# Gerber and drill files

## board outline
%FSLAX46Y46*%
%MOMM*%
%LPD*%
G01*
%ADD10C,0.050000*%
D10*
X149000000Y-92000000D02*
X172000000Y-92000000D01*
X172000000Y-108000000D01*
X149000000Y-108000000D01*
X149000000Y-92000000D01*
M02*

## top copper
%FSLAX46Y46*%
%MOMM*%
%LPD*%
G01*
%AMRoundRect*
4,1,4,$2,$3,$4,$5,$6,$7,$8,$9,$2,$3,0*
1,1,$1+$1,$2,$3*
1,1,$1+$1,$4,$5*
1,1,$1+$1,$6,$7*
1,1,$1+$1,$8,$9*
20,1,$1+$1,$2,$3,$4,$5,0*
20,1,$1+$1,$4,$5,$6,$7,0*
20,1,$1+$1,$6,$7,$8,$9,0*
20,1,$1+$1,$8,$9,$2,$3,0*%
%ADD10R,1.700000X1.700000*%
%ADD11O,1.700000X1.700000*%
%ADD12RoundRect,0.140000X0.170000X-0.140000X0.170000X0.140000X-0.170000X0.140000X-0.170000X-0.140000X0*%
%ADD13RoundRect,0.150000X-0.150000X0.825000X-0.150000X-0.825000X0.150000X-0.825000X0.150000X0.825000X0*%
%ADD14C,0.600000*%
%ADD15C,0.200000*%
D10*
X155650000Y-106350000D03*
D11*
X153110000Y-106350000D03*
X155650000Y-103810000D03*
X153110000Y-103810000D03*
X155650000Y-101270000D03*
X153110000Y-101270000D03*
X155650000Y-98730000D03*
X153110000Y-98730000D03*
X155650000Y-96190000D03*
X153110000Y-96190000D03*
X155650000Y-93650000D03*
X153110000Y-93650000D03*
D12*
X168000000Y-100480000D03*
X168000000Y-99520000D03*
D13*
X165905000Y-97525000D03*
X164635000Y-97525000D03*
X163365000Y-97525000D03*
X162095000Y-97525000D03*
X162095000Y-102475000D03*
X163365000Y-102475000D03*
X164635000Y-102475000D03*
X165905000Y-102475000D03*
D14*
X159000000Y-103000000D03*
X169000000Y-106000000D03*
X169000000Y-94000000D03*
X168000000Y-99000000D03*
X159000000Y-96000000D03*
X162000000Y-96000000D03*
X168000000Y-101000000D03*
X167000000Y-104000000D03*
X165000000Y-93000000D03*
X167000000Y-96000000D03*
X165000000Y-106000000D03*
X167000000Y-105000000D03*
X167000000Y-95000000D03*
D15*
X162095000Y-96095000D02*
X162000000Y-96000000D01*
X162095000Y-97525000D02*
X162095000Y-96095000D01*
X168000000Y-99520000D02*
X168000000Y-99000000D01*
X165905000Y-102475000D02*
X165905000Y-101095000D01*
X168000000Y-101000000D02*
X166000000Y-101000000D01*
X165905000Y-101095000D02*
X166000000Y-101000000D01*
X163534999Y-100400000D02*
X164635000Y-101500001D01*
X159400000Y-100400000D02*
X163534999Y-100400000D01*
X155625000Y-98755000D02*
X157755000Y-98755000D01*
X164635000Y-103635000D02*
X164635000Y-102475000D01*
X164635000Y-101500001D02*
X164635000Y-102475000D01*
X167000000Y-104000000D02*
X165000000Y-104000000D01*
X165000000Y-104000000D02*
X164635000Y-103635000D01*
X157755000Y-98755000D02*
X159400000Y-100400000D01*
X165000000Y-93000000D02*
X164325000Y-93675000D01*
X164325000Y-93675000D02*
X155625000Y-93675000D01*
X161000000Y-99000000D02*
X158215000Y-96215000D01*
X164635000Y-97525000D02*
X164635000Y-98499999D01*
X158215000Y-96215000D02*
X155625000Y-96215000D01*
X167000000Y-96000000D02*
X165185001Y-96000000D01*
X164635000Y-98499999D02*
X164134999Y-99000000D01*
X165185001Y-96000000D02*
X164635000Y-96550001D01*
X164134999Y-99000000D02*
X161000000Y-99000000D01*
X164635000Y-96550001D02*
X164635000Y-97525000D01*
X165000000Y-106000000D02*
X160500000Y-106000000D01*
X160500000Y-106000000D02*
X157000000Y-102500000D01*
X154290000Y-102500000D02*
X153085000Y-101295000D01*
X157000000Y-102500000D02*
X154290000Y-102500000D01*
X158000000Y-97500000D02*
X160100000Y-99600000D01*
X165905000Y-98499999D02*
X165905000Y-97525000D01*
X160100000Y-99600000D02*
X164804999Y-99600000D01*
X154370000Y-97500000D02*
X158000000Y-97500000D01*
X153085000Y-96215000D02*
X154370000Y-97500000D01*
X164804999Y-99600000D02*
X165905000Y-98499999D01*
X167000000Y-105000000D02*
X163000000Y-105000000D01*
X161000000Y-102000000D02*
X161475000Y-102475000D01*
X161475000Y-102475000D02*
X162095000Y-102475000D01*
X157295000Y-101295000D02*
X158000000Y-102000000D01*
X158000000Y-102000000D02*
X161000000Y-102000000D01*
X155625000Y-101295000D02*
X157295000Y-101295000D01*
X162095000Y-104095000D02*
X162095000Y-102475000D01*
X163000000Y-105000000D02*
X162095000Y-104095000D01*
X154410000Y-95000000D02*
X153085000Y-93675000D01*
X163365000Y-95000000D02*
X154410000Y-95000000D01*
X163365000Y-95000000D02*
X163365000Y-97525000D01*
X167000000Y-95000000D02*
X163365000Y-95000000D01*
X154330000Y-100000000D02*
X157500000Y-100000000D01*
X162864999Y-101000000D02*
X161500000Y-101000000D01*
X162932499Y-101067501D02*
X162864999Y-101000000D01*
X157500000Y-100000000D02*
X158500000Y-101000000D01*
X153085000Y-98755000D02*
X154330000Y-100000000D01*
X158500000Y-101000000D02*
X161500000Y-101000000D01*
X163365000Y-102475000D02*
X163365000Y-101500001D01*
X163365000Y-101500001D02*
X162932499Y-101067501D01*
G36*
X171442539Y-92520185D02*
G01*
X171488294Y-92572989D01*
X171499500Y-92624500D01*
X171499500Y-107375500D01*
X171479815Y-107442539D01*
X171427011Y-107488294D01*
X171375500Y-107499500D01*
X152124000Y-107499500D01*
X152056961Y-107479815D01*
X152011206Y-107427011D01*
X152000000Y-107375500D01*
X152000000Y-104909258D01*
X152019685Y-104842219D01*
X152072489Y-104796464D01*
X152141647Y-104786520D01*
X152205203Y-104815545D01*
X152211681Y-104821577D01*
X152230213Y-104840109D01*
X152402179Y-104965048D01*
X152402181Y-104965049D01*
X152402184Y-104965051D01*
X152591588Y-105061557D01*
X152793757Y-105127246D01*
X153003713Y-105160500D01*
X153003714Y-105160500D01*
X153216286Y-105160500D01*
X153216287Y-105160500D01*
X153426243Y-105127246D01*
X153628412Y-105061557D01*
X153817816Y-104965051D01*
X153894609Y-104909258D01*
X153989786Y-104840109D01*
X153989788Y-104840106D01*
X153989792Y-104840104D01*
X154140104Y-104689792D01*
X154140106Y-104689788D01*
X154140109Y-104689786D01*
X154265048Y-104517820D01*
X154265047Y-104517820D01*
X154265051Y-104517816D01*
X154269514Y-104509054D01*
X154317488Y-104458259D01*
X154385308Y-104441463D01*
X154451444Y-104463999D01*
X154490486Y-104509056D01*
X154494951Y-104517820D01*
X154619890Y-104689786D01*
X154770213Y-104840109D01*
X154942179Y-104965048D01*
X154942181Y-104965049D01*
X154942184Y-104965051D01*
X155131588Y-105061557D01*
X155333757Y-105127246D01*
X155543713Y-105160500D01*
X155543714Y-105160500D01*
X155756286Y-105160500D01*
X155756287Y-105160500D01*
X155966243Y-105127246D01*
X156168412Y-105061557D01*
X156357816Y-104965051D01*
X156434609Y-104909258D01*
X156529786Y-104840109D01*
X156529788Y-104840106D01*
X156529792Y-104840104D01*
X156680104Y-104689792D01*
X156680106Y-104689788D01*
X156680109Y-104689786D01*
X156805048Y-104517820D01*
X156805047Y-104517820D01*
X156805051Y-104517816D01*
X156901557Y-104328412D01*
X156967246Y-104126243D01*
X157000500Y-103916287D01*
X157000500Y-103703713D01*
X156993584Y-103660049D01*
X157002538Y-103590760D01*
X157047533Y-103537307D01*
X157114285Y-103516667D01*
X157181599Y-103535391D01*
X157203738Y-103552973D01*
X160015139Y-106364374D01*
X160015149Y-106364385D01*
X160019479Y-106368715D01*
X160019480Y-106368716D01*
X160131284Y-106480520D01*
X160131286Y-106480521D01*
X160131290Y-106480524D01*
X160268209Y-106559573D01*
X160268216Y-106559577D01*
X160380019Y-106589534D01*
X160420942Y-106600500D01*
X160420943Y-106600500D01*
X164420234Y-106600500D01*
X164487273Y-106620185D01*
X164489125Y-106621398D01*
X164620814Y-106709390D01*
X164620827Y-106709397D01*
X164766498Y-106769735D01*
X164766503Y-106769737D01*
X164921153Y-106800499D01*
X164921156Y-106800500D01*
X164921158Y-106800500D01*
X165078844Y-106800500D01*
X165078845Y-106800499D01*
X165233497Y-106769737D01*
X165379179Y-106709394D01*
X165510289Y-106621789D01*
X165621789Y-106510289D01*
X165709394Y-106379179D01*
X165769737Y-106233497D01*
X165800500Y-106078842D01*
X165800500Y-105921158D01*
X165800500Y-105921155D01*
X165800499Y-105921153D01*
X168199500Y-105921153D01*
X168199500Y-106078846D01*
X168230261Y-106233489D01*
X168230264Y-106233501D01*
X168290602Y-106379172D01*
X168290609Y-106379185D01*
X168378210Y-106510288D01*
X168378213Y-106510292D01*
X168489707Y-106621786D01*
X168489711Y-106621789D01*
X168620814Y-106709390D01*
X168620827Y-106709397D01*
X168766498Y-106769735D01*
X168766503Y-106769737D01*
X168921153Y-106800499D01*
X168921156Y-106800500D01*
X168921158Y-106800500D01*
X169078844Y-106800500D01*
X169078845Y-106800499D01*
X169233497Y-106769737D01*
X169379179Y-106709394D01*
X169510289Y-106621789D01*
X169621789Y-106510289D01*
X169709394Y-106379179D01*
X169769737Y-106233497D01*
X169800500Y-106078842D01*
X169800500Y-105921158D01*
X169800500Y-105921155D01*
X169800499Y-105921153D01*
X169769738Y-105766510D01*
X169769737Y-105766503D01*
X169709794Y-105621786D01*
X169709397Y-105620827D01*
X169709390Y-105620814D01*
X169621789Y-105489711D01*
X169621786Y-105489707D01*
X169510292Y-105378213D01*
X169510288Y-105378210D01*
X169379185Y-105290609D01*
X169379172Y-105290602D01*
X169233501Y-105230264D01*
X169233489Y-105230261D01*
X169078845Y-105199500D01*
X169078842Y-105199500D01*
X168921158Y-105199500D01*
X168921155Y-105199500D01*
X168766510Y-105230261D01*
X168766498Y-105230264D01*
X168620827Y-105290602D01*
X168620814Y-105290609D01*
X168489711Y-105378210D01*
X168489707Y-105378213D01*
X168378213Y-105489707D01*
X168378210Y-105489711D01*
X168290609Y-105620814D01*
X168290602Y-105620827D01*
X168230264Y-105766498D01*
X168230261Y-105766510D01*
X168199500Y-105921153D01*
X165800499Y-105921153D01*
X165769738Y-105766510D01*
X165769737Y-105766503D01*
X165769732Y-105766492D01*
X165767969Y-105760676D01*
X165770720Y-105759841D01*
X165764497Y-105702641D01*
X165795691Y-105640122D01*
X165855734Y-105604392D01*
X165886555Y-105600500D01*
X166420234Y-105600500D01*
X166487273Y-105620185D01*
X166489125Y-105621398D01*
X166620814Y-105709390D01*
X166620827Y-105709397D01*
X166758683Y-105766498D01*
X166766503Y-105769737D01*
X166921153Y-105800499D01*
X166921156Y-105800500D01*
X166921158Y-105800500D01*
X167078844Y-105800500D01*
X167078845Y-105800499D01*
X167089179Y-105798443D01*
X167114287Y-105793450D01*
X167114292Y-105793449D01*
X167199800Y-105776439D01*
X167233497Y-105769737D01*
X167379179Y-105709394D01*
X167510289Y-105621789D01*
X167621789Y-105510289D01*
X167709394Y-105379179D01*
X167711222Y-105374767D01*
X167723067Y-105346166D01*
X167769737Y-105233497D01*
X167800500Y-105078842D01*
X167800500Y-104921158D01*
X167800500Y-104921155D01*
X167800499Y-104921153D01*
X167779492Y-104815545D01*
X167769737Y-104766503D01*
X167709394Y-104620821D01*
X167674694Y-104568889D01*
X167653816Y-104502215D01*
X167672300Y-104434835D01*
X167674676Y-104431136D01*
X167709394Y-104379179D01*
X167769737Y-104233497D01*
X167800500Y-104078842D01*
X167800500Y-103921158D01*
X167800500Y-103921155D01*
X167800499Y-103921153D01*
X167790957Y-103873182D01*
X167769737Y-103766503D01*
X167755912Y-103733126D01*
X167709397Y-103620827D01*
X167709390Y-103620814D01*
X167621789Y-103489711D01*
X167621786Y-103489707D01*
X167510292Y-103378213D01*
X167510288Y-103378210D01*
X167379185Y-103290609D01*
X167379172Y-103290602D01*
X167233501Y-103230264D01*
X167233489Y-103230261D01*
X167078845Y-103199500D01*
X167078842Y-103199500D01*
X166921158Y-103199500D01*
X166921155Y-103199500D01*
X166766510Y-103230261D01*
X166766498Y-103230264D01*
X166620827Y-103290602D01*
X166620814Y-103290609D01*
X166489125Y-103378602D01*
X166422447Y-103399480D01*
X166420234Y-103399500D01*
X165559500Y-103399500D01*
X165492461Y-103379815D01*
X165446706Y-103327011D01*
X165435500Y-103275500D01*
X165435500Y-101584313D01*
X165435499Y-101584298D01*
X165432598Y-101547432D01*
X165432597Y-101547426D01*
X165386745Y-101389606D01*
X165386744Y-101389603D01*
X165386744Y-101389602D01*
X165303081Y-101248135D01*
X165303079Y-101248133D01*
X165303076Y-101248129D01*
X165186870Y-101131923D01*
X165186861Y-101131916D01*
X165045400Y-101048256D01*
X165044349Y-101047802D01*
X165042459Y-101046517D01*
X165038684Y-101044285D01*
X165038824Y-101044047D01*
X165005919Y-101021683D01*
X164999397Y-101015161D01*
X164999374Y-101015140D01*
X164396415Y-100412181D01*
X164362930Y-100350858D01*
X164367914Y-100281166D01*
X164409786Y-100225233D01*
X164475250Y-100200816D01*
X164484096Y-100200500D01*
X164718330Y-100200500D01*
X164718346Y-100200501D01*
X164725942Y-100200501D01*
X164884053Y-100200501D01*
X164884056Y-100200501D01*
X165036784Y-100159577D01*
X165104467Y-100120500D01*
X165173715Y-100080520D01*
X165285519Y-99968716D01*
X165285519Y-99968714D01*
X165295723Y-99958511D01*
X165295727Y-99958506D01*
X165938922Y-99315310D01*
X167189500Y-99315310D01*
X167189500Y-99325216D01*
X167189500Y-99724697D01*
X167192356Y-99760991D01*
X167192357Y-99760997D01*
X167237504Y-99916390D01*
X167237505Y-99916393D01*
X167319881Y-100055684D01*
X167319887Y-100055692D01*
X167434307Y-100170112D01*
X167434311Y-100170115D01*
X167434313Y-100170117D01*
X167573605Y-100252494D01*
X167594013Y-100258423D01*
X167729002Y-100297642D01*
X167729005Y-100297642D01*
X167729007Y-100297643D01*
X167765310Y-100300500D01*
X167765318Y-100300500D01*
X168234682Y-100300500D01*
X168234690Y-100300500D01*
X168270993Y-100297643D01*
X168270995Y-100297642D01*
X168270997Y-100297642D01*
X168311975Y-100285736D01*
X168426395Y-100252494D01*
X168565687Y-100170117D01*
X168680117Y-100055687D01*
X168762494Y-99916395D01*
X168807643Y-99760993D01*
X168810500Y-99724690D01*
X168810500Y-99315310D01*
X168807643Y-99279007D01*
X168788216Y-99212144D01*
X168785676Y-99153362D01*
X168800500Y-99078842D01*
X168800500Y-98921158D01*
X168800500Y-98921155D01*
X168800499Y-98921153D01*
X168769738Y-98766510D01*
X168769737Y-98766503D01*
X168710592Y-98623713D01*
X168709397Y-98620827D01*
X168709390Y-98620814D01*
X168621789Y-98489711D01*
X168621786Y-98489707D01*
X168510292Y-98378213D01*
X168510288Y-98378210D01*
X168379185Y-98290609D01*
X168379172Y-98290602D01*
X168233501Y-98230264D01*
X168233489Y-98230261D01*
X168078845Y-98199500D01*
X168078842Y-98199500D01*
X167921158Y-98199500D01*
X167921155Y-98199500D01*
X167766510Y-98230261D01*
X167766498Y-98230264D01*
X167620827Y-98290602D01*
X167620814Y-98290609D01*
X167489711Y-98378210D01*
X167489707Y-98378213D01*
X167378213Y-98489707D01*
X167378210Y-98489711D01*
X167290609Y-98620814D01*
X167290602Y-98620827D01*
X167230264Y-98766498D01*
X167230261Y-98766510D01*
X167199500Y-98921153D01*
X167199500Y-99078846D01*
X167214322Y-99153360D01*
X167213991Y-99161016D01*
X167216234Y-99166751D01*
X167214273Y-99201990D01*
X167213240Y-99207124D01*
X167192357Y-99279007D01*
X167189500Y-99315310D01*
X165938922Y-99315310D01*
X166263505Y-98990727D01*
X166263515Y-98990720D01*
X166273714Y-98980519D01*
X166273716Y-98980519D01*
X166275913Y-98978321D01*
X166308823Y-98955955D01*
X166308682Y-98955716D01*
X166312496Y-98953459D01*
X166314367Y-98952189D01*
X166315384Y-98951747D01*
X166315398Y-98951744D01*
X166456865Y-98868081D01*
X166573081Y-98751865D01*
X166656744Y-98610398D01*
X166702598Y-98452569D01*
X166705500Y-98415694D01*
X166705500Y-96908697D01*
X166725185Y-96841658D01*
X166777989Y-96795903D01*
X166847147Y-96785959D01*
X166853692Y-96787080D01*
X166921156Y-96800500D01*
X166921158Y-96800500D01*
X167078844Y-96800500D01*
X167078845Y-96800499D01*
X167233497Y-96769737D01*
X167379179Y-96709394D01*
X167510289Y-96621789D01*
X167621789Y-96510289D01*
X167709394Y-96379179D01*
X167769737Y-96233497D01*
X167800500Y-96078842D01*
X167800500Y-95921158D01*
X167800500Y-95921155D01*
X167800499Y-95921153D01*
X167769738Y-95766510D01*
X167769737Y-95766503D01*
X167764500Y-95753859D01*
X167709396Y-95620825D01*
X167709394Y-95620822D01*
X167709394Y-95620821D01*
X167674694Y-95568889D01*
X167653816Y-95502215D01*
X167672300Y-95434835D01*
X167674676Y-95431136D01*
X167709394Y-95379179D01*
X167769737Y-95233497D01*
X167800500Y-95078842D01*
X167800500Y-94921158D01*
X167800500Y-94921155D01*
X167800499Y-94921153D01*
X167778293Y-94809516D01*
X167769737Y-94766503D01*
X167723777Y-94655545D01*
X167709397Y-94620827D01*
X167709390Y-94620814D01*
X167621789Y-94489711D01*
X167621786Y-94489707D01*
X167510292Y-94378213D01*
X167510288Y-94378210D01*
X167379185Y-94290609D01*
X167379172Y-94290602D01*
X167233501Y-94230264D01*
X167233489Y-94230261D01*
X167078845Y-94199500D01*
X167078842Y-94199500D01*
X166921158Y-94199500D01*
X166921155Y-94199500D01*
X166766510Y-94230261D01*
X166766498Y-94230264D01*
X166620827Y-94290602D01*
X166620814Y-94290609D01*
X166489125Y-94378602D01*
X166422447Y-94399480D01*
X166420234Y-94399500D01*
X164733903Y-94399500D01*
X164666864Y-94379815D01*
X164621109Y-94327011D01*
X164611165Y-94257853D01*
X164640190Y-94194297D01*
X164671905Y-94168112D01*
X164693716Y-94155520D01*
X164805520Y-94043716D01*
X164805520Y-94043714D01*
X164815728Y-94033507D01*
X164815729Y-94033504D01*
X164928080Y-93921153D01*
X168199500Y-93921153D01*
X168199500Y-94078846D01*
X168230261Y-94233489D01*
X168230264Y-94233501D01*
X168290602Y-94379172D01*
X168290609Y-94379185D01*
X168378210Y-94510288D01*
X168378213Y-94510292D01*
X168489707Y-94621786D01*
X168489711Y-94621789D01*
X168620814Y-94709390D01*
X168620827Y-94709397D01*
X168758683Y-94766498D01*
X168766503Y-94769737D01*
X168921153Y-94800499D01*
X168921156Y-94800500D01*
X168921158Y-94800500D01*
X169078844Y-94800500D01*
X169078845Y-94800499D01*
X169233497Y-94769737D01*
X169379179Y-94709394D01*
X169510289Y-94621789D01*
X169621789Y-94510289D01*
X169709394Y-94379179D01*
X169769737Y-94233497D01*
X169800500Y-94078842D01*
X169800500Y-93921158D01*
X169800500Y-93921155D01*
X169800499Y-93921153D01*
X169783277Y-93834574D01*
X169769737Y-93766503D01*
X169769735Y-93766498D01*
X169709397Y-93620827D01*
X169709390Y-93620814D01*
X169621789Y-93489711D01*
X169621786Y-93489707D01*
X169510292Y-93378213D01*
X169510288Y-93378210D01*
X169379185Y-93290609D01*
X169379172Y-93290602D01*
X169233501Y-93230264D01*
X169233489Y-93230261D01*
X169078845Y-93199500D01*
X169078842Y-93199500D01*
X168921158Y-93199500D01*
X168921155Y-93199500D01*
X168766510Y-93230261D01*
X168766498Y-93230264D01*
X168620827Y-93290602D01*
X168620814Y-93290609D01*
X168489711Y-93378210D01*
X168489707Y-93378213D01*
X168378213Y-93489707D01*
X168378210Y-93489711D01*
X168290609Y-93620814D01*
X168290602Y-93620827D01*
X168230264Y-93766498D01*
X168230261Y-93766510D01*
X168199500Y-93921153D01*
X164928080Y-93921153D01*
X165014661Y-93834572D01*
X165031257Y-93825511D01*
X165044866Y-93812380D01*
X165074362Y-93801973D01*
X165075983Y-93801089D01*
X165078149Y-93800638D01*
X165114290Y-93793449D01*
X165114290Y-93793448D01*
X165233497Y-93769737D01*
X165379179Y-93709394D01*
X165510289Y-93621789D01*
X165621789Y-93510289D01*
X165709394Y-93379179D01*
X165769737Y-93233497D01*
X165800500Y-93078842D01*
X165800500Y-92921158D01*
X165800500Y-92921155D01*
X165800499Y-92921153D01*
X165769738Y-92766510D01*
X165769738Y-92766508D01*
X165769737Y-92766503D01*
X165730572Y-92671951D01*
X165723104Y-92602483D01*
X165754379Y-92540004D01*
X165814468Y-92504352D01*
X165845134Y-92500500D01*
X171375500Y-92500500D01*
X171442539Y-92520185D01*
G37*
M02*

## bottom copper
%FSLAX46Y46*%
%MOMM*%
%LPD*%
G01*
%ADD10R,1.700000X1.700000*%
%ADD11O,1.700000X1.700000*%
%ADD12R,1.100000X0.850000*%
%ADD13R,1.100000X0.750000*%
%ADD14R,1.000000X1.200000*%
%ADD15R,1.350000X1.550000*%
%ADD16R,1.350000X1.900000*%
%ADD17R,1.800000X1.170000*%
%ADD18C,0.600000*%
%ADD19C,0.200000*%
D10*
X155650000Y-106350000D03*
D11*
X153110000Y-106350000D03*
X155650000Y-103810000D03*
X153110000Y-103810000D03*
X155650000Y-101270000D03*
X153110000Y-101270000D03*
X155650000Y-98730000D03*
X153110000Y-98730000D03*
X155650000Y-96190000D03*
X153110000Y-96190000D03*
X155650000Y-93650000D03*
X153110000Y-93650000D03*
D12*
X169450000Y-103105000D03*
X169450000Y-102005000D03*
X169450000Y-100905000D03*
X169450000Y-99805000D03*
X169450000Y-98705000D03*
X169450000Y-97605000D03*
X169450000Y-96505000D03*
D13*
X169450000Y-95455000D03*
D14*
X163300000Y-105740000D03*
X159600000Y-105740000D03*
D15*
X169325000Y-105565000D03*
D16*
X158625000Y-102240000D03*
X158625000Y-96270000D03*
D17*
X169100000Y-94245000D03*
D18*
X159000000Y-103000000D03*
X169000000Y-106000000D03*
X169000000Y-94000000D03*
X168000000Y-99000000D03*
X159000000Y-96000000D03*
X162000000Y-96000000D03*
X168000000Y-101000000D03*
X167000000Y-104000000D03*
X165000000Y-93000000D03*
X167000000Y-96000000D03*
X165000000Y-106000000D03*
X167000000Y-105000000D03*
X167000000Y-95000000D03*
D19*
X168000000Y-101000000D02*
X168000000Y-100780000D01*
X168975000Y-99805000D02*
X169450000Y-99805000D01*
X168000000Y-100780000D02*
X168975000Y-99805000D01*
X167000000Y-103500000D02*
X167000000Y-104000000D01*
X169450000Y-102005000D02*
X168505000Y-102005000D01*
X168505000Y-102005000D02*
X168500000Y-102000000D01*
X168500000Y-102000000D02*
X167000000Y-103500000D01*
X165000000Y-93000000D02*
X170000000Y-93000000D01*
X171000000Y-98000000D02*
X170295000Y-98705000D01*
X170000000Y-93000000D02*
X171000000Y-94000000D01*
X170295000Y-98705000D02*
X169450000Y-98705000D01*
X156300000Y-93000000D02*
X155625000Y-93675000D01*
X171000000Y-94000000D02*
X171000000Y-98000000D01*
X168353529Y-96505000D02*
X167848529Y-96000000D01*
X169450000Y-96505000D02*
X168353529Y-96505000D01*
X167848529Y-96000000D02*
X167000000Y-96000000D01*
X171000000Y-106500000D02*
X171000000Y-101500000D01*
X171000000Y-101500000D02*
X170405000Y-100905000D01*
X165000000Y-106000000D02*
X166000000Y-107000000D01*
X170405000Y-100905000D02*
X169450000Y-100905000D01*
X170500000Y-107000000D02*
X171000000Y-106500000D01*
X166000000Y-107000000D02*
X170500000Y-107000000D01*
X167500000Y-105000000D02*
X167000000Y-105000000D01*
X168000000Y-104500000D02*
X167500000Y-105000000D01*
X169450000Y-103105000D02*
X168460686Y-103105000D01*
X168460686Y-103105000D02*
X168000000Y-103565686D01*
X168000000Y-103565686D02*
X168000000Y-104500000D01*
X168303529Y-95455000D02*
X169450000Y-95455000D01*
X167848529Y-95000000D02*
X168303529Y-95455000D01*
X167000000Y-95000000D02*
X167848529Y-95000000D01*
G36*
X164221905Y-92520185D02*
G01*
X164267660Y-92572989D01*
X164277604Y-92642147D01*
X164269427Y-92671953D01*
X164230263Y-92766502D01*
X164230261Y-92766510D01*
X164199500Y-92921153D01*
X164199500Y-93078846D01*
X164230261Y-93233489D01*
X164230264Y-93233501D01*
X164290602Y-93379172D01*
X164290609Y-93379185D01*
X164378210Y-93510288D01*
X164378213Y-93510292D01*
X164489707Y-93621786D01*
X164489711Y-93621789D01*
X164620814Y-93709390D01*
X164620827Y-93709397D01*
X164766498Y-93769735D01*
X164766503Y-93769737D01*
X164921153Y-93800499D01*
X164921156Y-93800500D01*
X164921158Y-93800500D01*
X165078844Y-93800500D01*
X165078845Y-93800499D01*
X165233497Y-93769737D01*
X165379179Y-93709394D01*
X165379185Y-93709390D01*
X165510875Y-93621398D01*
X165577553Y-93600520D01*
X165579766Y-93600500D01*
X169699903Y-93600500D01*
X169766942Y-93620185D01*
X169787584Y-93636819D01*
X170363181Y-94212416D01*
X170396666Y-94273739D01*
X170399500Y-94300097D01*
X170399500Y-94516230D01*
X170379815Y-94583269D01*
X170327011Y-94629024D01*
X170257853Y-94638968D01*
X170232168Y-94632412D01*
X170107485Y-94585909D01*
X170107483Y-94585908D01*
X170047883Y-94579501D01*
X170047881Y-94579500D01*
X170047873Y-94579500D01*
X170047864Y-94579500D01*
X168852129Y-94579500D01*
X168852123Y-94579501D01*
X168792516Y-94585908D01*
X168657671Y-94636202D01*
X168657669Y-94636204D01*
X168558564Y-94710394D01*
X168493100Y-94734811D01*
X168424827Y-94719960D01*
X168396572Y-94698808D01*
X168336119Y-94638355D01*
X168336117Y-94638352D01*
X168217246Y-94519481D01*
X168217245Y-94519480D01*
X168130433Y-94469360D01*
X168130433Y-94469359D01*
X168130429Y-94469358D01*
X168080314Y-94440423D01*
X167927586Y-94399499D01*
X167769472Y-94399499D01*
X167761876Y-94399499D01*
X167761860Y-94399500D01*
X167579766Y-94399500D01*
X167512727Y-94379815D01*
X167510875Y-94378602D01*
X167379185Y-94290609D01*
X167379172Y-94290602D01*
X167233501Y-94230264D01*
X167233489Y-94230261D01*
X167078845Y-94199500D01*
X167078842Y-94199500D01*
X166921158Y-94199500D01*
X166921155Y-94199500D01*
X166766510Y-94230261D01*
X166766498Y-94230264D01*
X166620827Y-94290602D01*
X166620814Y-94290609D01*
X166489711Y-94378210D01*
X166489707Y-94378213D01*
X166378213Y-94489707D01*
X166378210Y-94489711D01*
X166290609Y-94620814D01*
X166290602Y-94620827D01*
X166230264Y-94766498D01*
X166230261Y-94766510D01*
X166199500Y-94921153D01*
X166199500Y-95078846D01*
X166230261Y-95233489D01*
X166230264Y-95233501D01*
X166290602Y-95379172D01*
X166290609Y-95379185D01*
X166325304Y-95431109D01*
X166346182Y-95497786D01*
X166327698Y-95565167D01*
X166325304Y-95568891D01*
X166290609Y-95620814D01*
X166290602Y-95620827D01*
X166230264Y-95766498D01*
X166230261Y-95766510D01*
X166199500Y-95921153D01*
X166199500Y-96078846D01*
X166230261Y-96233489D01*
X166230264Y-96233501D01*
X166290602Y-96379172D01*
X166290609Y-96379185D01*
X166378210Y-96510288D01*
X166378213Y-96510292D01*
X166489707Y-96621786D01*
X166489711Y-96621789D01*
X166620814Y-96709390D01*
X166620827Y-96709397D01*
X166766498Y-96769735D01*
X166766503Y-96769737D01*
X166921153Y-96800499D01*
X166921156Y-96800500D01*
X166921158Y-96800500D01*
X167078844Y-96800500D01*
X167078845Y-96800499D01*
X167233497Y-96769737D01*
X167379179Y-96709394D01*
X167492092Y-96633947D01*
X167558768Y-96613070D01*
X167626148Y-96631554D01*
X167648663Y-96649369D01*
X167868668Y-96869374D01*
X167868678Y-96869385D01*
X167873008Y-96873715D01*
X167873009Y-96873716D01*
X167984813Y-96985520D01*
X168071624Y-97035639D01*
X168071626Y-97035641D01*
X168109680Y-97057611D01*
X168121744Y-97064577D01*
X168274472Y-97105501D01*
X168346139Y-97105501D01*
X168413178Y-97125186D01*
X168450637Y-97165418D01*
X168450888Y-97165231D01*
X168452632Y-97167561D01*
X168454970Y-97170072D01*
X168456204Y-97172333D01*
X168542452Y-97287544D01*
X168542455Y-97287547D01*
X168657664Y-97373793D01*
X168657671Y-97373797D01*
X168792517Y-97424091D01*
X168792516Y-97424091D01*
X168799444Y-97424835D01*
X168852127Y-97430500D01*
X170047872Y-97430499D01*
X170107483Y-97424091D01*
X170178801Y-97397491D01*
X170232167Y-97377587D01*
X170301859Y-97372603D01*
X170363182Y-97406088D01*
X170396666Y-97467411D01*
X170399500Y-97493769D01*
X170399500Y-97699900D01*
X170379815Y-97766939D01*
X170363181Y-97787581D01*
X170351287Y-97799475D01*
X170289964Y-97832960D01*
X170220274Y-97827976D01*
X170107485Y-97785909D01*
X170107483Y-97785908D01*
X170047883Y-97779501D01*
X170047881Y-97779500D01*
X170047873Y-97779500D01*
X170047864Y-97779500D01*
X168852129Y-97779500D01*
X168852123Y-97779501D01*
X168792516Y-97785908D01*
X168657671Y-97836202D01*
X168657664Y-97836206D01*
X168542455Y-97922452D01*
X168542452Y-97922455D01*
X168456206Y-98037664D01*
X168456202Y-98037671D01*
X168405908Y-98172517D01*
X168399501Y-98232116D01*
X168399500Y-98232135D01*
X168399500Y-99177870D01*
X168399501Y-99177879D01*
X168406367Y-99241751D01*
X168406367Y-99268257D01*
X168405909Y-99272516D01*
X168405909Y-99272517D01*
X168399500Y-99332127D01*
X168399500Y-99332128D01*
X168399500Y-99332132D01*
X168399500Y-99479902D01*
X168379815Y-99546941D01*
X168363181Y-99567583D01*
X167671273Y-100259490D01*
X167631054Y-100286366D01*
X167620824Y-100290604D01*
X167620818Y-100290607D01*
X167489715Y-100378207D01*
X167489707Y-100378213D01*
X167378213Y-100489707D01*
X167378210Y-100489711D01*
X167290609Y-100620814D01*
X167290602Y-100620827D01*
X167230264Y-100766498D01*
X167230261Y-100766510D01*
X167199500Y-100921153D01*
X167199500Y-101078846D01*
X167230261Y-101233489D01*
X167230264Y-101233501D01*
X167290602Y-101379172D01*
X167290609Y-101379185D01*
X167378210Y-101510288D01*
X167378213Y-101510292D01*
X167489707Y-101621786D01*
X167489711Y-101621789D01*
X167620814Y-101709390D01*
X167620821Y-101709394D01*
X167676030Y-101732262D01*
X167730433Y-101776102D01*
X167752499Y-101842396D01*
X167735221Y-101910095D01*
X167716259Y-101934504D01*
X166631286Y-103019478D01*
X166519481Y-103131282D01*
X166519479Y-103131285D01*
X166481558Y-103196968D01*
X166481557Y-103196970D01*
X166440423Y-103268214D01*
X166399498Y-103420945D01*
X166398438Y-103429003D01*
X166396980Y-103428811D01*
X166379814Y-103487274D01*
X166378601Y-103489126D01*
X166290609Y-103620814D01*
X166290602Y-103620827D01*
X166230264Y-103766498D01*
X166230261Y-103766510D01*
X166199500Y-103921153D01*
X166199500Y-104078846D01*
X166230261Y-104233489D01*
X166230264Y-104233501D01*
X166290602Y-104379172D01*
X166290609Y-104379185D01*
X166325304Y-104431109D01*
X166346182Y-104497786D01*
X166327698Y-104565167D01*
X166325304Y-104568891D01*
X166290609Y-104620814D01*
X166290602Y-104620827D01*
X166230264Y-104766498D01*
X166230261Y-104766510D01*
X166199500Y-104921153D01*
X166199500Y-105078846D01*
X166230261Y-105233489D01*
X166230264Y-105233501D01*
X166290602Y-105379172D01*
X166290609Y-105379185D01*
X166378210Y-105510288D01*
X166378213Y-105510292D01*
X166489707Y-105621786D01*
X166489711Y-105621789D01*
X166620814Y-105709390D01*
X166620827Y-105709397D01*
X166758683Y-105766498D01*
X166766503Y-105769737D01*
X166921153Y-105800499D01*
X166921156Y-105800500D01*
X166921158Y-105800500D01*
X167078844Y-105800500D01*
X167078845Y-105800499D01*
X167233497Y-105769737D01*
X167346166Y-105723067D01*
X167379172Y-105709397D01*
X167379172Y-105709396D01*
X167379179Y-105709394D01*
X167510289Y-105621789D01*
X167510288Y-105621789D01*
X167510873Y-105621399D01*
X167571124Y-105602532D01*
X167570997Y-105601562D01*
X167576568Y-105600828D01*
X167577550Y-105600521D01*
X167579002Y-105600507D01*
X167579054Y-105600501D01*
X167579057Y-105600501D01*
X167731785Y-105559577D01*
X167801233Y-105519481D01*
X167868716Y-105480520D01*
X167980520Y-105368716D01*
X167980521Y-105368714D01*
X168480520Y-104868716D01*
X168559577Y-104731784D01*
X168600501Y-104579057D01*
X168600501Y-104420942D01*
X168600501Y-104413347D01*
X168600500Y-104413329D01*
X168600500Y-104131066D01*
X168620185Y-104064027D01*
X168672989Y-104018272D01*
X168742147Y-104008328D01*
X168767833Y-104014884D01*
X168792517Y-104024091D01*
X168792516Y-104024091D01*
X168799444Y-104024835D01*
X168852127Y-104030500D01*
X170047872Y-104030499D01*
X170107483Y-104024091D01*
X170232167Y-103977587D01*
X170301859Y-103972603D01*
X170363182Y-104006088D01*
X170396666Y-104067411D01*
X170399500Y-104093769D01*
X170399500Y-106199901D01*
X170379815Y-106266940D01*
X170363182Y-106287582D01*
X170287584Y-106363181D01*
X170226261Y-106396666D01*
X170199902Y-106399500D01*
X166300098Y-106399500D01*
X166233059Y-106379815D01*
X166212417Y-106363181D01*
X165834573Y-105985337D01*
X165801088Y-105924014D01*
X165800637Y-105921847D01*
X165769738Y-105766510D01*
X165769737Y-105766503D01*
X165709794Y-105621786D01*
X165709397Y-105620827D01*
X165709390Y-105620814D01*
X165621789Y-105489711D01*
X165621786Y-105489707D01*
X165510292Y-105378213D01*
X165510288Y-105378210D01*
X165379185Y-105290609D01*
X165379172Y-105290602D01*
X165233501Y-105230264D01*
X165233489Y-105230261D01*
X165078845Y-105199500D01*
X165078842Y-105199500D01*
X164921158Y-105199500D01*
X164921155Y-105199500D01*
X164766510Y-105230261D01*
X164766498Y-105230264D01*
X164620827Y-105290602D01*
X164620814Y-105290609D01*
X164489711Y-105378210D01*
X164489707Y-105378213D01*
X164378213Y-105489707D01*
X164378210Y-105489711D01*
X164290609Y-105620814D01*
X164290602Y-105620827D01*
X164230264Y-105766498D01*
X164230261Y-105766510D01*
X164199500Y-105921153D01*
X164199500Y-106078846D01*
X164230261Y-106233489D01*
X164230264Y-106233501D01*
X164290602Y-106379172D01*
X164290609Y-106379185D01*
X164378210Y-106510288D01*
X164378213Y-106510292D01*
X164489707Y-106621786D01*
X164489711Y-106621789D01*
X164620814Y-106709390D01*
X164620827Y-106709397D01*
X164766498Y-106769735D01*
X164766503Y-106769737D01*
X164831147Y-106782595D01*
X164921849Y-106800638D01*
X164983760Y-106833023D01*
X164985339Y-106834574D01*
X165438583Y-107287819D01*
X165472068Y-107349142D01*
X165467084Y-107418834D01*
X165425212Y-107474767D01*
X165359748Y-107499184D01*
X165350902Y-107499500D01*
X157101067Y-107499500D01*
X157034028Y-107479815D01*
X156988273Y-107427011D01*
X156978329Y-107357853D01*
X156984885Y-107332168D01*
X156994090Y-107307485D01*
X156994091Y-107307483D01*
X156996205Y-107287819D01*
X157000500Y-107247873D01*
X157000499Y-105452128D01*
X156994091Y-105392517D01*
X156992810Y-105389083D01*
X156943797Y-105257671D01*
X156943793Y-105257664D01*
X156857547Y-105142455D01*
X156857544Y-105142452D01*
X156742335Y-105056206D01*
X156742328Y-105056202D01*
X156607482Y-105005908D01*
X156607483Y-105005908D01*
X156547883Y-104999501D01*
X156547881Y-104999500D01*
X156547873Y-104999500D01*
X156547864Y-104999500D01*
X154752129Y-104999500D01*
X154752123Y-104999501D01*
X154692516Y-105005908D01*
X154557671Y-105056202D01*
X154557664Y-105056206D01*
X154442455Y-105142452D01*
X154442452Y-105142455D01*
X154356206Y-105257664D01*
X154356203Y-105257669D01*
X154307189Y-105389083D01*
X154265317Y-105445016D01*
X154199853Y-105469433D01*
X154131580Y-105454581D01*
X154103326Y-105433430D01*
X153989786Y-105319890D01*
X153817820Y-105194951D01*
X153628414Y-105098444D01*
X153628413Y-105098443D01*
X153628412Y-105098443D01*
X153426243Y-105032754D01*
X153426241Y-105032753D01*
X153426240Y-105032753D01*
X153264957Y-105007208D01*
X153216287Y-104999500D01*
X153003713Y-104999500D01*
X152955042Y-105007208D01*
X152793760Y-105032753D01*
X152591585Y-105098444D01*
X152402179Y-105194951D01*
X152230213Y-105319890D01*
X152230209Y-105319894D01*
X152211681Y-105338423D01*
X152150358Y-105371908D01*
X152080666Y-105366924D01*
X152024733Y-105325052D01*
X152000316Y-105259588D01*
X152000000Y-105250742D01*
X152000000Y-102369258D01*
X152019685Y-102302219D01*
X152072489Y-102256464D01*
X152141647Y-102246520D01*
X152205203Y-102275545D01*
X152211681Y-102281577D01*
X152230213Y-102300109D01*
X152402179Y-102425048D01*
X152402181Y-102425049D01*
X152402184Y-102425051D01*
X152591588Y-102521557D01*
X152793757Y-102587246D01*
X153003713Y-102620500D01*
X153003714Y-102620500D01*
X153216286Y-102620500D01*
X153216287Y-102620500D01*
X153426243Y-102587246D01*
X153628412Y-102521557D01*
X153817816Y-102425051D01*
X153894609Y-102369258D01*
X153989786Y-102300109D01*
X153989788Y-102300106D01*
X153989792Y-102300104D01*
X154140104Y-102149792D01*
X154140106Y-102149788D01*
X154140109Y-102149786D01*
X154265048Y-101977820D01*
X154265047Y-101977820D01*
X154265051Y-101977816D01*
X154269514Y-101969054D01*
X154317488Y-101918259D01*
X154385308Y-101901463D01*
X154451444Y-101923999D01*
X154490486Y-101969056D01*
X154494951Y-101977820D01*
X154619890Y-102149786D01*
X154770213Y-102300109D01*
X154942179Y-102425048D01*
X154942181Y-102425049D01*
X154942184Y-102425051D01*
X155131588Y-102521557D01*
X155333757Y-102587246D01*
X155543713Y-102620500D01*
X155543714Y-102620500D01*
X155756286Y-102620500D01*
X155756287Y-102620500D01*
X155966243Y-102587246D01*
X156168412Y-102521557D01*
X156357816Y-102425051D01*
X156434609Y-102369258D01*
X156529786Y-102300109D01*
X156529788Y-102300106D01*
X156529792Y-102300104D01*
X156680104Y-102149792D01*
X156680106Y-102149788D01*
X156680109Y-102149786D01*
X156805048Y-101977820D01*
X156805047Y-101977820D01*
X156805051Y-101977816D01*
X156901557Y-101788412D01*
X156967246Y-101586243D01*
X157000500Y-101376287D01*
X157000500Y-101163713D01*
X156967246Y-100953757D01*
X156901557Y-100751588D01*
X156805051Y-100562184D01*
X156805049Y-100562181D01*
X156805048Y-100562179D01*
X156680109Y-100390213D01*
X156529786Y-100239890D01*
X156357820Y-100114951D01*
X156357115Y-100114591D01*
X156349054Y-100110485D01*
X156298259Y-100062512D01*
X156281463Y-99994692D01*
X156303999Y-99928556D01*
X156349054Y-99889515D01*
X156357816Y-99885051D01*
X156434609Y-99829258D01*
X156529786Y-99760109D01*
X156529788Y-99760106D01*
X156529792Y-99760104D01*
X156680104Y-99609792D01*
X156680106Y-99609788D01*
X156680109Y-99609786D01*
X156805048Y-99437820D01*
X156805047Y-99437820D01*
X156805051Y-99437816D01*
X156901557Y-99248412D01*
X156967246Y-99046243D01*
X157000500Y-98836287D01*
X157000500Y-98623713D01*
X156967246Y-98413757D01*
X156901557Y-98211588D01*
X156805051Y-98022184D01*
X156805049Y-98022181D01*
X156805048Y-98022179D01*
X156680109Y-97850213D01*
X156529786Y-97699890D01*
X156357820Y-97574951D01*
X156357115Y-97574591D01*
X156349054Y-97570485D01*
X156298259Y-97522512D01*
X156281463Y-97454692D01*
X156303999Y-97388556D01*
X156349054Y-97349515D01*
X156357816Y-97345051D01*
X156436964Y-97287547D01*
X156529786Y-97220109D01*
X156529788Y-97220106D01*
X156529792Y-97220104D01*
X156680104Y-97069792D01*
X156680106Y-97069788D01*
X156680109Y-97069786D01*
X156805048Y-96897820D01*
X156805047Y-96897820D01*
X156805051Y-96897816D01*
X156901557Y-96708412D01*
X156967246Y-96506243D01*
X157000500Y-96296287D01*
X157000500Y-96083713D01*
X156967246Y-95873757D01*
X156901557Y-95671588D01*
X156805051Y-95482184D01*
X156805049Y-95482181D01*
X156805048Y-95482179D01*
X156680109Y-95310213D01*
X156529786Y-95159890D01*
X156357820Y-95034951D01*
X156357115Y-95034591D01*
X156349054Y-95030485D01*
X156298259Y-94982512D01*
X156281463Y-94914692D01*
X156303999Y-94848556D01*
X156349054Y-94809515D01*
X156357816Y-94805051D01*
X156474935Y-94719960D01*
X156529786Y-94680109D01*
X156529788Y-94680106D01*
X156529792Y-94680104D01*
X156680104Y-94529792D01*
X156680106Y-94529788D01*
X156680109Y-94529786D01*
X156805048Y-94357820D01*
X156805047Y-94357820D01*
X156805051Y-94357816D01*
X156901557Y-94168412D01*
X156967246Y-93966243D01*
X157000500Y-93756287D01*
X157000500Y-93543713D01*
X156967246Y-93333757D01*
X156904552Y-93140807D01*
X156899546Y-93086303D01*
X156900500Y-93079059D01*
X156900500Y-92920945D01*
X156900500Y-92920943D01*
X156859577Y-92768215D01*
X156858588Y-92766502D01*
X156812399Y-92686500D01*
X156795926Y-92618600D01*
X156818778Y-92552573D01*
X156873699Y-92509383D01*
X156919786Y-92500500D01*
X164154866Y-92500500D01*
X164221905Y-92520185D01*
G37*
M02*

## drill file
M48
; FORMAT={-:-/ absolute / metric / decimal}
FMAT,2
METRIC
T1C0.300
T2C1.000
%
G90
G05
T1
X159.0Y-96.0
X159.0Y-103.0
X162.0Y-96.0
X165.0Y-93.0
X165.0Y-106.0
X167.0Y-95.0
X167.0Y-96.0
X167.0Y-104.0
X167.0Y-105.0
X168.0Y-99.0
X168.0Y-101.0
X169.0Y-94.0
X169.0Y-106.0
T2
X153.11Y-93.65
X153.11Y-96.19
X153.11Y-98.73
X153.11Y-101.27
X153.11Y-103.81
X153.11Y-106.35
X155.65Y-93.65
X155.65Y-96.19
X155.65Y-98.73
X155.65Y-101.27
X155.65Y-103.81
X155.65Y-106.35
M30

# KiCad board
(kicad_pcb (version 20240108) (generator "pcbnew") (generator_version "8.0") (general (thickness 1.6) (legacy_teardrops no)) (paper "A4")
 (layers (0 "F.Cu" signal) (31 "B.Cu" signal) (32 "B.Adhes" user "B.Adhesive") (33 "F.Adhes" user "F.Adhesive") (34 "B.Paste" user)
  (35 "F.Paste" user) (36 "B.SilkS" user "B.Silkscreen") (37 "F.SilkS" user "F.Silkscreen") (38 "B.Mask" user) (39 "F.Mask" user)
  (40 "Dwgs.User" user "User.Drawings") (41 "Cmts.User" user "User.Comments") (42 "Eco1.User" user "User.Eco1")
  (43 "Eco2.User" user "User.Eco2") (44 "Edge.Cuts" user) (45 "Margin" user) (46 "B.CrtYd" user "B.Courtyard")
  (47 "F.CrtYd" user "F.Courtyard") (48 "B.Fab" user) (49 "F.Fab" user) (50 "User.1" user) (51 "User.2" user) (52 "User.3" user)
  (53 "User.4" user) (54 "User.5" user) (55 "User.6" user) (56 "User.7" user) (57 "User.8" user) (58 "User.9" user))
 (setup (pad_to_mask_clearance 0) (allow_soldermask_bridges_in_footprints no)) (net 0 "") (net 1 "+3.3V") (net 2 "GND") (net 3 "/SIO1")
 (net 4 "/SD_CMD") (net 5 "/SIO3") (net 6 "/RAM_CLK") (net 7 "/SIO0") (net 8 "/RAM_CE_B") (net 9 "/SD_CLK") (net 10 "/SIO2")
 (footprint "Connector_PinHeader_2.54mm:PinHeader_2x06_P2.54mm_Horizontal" (layer "F.Cu") (at 155.65 106.35 180)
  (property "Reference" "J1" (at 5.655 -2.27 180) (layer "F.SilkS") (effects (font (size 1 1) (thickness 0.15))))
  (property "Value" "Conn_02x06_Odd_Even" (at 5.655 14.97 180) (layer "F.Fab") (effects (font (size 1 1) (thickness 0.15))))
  (pad "1" thru_hole rect (at 0 0 180) (size 1.7 1.7) (drill 1) (layers "*.Cu" "*.Mask") (remove_unused_layers no) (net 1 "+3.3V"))
  (pad "2" thru_hole oval (at 2.54 0 180) (size 1.7 1.7) (drill 1) (layers "*.Cu" "*.Mask") (remove_unused_layers no) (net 1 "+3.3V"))
  (pad "3" thru_hole oval (at 0 2.54 180) (size 1.7 1.7) (drill 1) (layers "*.Cu" "*.Mask") (remove_unused_layers no) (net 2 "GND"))
  (pad "4" thru_hole oval (at 2.54 2.54 180) (size 1.7 1.7) (drill 1) (layers "*.Cu" "*.Mask") (remove_unused_layers no) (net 2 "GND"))
  (pad "5" thru_hole oval (at 0 5.08 180) (size 1.7 1.7) (drill 1) (layers "*.Cu" "*.Mask") (remove_unused_layers no) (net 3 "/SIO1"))
  (pad "6" thru_hole oval (at 2.54 5.08 180) (size 1.7 1.7) (drill 1) (layers "*.Cu" "*.Mask") (remove_unused_layers no) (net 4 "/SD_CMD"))
  (pad "7" thru_hole oval (at 0 7.62 180) (size 1.7 1.7) (drill 1) (layers "*.Cu" "*.Mask") (remove_unused_layers no) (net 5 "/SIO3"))
  (pad "8" thru_hole oval (at 2.54 7.62 180) (size 1.7 1.7) (drill 1) (layers "*.Cu" "*.Mask") (remove_unused_layers no) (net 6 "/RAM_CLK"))
  (pad "9" thru_hole oval (at 0 10.16 180) (size 1.7 1.7) (drill 1) (layers "*.Cu" "*.Mask") (remove_unused_layers no) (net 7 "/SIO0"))
  (pad "10" thru_hole oval (at 2.54 10.16 180) (size 1.7 1.7) (drill 1) (layers "*.Cu" "*.Mask") (remove_unused_layers no)
   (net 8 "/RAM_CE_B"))
  (pad "11" thru_hole oval (at 0 12.7 180) (size 1.7 1.7) (drill 1) (layers "*.Cu" "*.Mask") (remove_unused_layers no) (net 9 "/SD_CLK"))
  (pad "12" thru_hole oval (at 2.54 12.7 180) (size 1.7 1.7) (drill 1) (layers "*.Cu" "*.Mask") (remove_unused_layers no) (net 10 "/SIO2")))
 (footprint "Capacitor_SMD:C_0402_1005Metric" (layer "F.Cu") (at 168 100 90)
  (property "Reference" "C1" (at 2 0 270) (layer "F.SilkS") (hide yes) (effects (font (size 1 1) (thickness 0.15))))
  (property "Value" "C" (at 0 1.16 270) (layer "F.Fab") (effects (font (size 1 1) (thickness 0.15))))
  (pad "1" smd roundrect (at -0.48 0 90) (size 0.56 0.62) (layers "F.Cu" "F.Paste" "F.Mask") (roundrect_rratio 0.25) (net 1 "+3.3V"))
  (pad "2" smd roundrect (at 0.48 0 90) (size 0.56 0.62) (layers "F.Cu" "F.Paste" "F.Mask") (roundrect_rratio 0.25) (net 2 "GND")))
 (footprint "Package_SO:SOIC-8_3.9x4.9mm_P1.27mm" (layer "F.Cu") (at 164 100 -90)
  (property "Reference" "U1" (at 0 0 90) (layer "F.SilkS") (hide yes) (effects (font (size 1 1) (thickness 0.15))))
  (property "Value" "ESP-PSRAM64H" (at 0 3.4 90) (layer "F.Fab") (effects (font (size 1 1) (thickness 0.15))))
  (pad "1" smd roundrect (at -2.475 -1.905 270) (size 1.95 0.6) (layers "F.Cu" "F.Paste" "F.Mask") (roundrect_rratio 0.25)
   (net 8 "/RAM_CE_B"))
  (pad "2" smd roundrect (at -2.475 -0.635 270) (size 1.95 0.6) (layers "F.Cu" "F.Paste" "F.Mask") (roundrect_rratio 0.25) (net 7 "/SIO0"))
  (pad "3" smd roundrect (at -2.475 0.635 270) (size 1.95 0.6) (layers "F.Cu" "F.Paste" "F.Mask") (roundrect_rratio 0.25) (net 10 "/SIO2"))
  (pad "4" smd roundrect (at -2.475 1.905 270) (size 1.95 0.6) (layers "F.Cu" "F.Paste" "F.Mask") (roundrect_rratio 0.25) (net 2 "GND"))
  (pad "5" smd roundrect (at 2.475 1.905 270) (size 1.95 0.6) (layers "F.Cu" "F.Paste" "F.Mask") (roundrect_rratio 0.25) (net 3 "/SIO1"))
  (pad "6" smd roundrect (at 2.475 0.635 270) (size 1.95 0.6) (layers "F.Cu" "F.Paste" "F.Mask") (roundrect_rratio 0.25) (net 6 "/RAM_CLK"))
  (pad "7" smd roundrect (at 2.475 -0.635 270) (size 1.95 0.6) (layers "F.Cu" "F.Paste" "F.Mask") (roundrect_rratio 0.25) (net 5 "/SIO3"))
  (pad "8" smd roundrect (at 2.475 -1.905 270) (size 1.95 0.6) (layers "F.Cu" "F.Paste" "F.Mask") (roundrect_rratio 0.25) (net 1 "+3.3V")))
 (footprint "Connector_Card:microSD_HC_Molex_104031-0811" (layer "B.Cu") (at 164 100 90)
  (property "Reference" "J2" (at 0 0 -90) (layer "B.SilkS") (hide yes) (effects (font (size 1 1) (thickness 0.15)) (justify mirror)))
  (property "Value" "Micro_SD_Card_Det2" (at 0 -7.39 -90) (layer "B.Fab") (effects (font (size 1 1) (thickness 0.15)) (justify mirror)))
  (pad "1" smd rect (at -3.105 5.45 90) (size 0.85 1.1) (layers "B.Cu" "B.Paste" "B.Mask") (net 3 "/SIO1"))
  (pad "2" smd rect (at -2.005 5.45 90) (size 0.85 1.1) (layers "B.Cu" "B.Paste" "B.Mask") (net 5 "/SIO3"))
  (pad "3" smd rect (at -0.905 5.45 90) (size 0.85 1.1) (layers "B.Cu" "B.Paste" "B.Mask") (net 4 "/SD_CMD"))
  (pad "4" smd rect (at 0.195 5.45 90) (size 0.85 1.1) (layers "B.Cu" "B.Paste" "B.Mask") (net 1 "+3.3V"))
  (pad "5" smd rect (at 1.295 5.45 90) (size 0.85 1.1) (layers "B.Cu" "B.Paste" "B.Mask") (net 9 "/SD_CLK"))
  (pad "6" smd rect (at 2.395 5.45 90) (size 0.85 1.1) (layers "B.Cu" "B.Paste" "B.Mask") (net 2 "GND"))
  (pad "7" smd rect (at 3.495 5.45 90) (size 0.85 1.1) (layers "B.Cu" "B.Paste" "B.Mask") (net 7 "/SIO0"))
  (pad "8" smd rect (at 4.545 5.45 90) (size 0.75 1.1) (layers "B.Cu" "B.Paste" "B.Mask") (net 10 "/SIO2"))
  (pad "9" smd rect (at -5.74 -0.7 90) (size 1.2 1) (layers "B.Cu" "B.Paste" "B.Mask") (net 2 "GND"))
  (pad "10" smd rect (at -5.74 -4.4 90) (size 1.2 1) (layers "B.Cu" "B.Paste" "B.Mask") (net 2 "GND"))
  (pad "11" smd rect (at -5.565 5.325 90) (size 1.55 1.35) (layers "B.Cu" "B.Paste" "B.Mask") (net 2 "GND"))
  (pad "11" smd rect (at -2.24 -5.375 90) (size 1.9 1.35) (layers "B.Cu" "B.Paste" "B.Mask") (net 2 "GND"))
  (pad "11" smd rect (at 3.73 -5.375 90) (size 1.9 1.35) (layers "B.Cu" "B.Paste" "B.Mask") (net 2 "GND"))
  (pad "11" smd rect (at 5.755 5.1 90) (size 1.17 1.8) (layers "B.Cu" "B.Paste" "B.Mask") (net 2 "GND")))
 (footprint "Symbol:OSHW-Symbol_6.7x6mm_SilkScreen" (layer "B.Cu") (at 164 100 180)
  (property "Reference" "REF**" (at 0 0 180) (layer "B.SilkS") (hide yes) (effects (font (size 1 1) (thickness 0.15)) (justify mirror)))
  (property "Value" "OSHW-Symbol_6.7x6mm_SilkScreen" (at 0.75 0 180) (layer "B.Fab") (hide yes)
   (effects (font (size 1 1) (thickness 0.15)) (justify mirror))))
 (gr_rect (start 149 92) (end 172 108) (stroke (width 0.05) (type default)) (fill none) (layer "Edge.Cuts"))
 (segment (start 162.095 96.095) (end 162 96) (width 0.2) (layer "F.Cu") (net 2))
 (segment (start 162.095 97.525) (end 162.095 96.095) (width 0.2) (layer "F.Cu") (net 2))
 (segment (start 168 99.52) (end 168 99) (width 0.2) (layer "F.Cu") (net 2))
 (via (at 159 103) (size 0.6) (drill 0.3) (layers "F.Cu" "B.Cu") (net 2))
 (via (at 169 106) (size 0.6) (drill 0.3) (layers "F.Cu" "B.Cu") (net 2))
 (via (at 169 94) (size 0.6) (drill 0.3) (layers "F.Cu" "B.Cu") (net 2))
 (via (at 168 99) (size 0.6) (drill 0.3) (layers "F.Cu" "B.Cu") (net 2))
 (via (at 159 96) (size 0.6) (drill 0.3) (layers "F.Cu" "B.Cu") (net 2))
 (via (at 162 96) (size 0.6) (drill 0.3) (layers "F.Cu" "B.Cu") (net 2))
 (segment (start 165.905 102.475) (end 165.905 101.095) (width 0.2) (layer "F.Cu") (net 1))
 (segment (start 168 101) (end 166 101) (width 0.2) (layer "F.Cu") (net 1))
 (segment (start 165.905 101.095) (end 166 101) (width 0.2) (layer "F.Cu") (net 1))
 (via (at 168 101) (size 0.6) (drill 0.3) (layers "F.Cu" "B.Cu") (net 1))
 (segment (start 168 101) (end 168 100.78) (width 0.2) (layer "B.Cu") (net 1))
 (segment (start 168.975 99.805) (end 169.45 99.805) (width 0.2) (layer "B.Cu") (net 1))
 (segment (start 168 100.78) (end 168.975 99.805) (width 0.2) (layer "B.Cu") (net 1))
 (segment (start 163.534999 100.4) (end 164.635 101.500001) (width 0.2) (layer "F.Cu") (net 5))
 (segment (start 159.4 100.4) (end 163.534999 100.4) (width 0.2) (layer "F.Cu") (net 5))
 (segment (start 155.625 98.755) (end 157.755 98.755) (width 0.2) (layer "F.Cu") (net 5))
 (segment (start 164.635 103.635) (end 164.635 102.475) (width 0.2) (layer "F.Cu") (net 5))
 (segment (start 164.635 101.500001) (end 164.635 102.475) (width 0.2) (layer "F.Cu") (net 5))
 (segment (start 167 104) (end 165 104) (width 0.2) (layer "F.Cu") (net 5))
 (segment (start 165 104) (end 164.635 103.635) (width 0.2) (layer "F.Cu") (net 5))
 (segment (start 157.755 98.755) (end 159.4 100.4) (width 0.2) (layer "F.Cu") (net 5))
 (via (at 167 104) (size 0.6) (drill 0.3) (layers "F.Cu" "B.Cu") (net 5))
 (segment (start 167 103.5) (end 167 104) (width 0.2) (layer "B.Cu") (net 5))
 (segment (start 169.45 102.005) (end 168.505 102.005) (width 0.2) (layer "B.Cu") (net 5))
 (segment (start 168.505 102.005) (end 168.5 102) (width 0.2) (layer "B.Cu") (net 5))
 (segment (start 168.5 102) (end 167 103.5) (width 0.2) (layer "B.Cu") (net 5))
 (segment (start 165 93) (end 164.325 93.675) (width 0.2) (layer "F.Cu") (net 9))
 (segment (start 164.325 93.675) (end 155.625 93.675) (width 0.2) (layer "F.Cu") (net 9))
 (via (at 165 93) (size 0.6) (drill 0.3) (layers "F.Cu" "B.Cu") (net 9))
 (segment (start 165 93) (end 170 93) (width 0.2) (layer "B.Cu") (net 9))
 (segment (start 171 98) (end 170.295 98.705) (width 0.2) (layer "B.Cu") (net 9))
 (segment (start 170 93) (end 171 94) (width 0.2) (layer "B.Cu") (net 9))
 (segment (start 170.295 98.705) (end 169.45 98.705) (width 0.2) (layer "B.Cu") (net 9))
 (segment (start 156.3 93) (end 155.625 93.675) (width 0.2) (layer "B.Cu") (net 9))
 (segment (start 171 94) (end 171 98) (width 0.2) (layer "B.Cu") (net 9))
 (segment (start 161 99) (end 158.215 96.215) (width 0.2) (layer "F.Cu") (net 7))
 (segment (start 164.635 97.525) (end 164.635 98.499999) (width 0.2) (layer "F.Cu") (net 7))
 (segment (start 158.215 96.215) (end 155.625 96.215) (width 0.2) (layer "F.Cu") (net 7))
 (segment (start 167 96) (end 165.185001 96) (width 0.2) (layer "F.Cu") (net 7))
 (segment (start 164.635 98.499999) (end 164.134999 99) (width 0.2) (layer "F.Cu") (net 7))
 (segment (start 165.185001 96) (end 164.635 96.550001) (width 0.2) (layer "F.Cu") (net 7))
 (segment (start 164.134999 99) (end 161 99) (width 0.2) (layer "F.Cu") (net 7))
 (segment (start 164.635 96.550001) (end 164.635 97.525) (width 0.2) (layer "F.Cu") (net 7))
 (via (at 167 96) (size 0.6) (drill 0.3) (layers "F.Cu" "B.Cu") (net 7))
 (segment (start 168.353529 96.505) (end 167.848529 96) (width 0.2) (layer "B.Cu") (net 7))
 (segment (start 169.45 96.505) (end 168.353529 96.505) (width 0.2) (layer "B.Cu") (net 7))
 (segment (start 167.848529 96) (end 167 96) (width 0.2) (layer "B.Cu") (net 7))
 (segment (start 165 106) (end 160.5 106) (width 0.2) (layer "F.Cu") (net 4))
 (segment (start 160.5 106) (end 157 102.5) (width 0.2) (layer "F.Cu") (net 4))
 (segment (start 154.29 102.5) (end 153.085 101.295) (width 0.2) (layer "F.Cu") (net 4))
 (segment (start 157 102.5) (end 154.29 102.5) (width 0.2) (layer "F.Cu") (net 4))
 (via (at 165 106) (size 0.6) (drill 0.3) (layers "F.Cu" "B.Cu") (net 4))
 (segment (start 171 106.5) (end 171 101.5) (width 0.2) (layer "B.Cu") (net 4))
 (segment (start 171 101.5) (end 170.405 100.905) (width 0.2) (layer "B.Cu") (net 4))
 (segment (start 165 106) (end 166 107) (width 0.2) (layer "B.Cu") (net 4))
 (segment (start 170.405 100.905) (end 169.45 100.905) (width 0.2) (layer "B.Cu") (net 4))
 (segment (start 170.5 107) (end 171 106.5) (width 0.2) (layer "B.Cu") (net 4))
 (segment (start 166 107) (end 170.5 107) (width 0.2) (layer "B.Cu") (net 4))
 (segment (start 158 97.5) (end 160.1 99.6) (width 0.2) (layer "F.Cu") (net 8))
 (segment (start 165.905 98.499999) (end 165.905 97.525) (width 0.2) (layer "F.Cu") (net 8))
 (segment (start 160.1 99.6) (end 164.804999 99.6) (width 0.2) (layer "F.Cu") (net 8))
 (segment (start 154.37 97.5) (end 158 97.5) (width 0.2) (layer "F.Cu") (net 8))
 (segment (start 153.085 96.215) (end 154.37 97.5) (width 0.2) (layer "F.Cu") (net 8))
 (segment (start 164.804999 99.6) (end 165.905 98.499999) (width 0.2) (layer "F.Cu") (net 8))
 (segment (start 167 105) (end 163 105) (width 0.2) (layer "F.Cu") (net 3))
 (segment (start 161 102) (end 161.475 102.475) (width 0.2) (layer "F.Cu") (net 3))
 (segment (start 161.475 102.475) (end 162.095 102.475) (width 0.2) (layer "F.Cu") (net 3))
 (segment (start 157.295 101.295) (end 158 102) (width 0.2) (layer "F.Cu") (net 3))
 (segment (start 158 102) (end 161 102) (width 0.2) (layer "F.Cu") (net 3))
 (segment (start 155.625 101.295) (end 157.295 101.295) (width 0.2) (layer "F.Cu") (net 3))
 (segment (start 162.095 104.095) (end 162.095 102.475) (width 0.2) (layer "F.Cu") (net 3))
 (segment (start 163 105) (end 162.095 104.095) (width 0.2) (layer "F.Cu") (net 3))
 (via (at 167 105) (size 0.6) (drill 0.3) (layers "F.Cu" "B.Cu") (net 3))
 (segment (start 167.5 105) (end 167 105) (width 0.2) (layer "B.Cu") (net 3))
 (segment (start 168 104.5) (end 167.5 105) (width 0.2) (layer "B.Cu") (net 3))
 (segment (start 169.45 103.105) (end 168.460686 103.105) (width 0.2) (layer "B.Cu") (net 3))
 (segment (start 168.460686 103.105) (end 168 103.565686) (width 0.2) (layer "B.Cu") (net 3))
 (segment (start 168 103.565686) (end 168 104.5) (width 0.2) (layer "B.Cu") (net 3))
 (segment (start 154.41 95) (end 153.085 93.675) (width 0.2) (layer "F.Cu") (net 10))
 (segment (start 163.365 95) (end 154.41 95) (width 0.2) (layer "F.Cu") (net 10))
 (segment (start 163.365 95) (end 163.365 97.525) (width 0.2) (layer "F.Cu") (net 10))
 (segment (start 167 95) (end 163.365 95) (width 0.2) (layer "F.Cu") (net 10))
 (via (at 167 95) (size 0.6) (drill 0.3) (layers "F.Cu" "B.Cu") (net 10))
 (segment (start 168.303529 95.455) (end 169.45 95.455) (width 0.2) (layer "B.Cu") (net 10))
 (segment (start 167.848529 95) (end 168.303529 95.455) (width 0.2) (layer "B.Cu") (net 10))
 (segment (start 167 95) (end 167.848529 95) (width 0.2) (layer "B.Cu") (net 10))
 (segment (start 154.33 100) (end 157.5 100) (width 0.2) (layer "F.Cu") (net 6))
 (segment (start 162.864999 101) (end 161.5 101) (width 0.2) (layer "F.Cu") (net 6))
 (segment (start 162.932499 101.067501) (end 162.864999 101) (width 0.2) (layer "F.Cu") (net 6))
 (segment (start 157.5 100) (end 158.5 101) (width 0.2) (layer "F.Cu") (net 6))
 (segment (start 153.085 98.755) (end 154.33 100) (width 0.2) (layer "F.Cu") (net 6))
 (segment (start 158.5 101) (end 161.5 101) (width 0.2) (layer "F.Cu") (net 6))
 (segment (start 163.365 102.475) (end 163.365 101.500001) (width 0.2) (layer "F.Cu") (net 6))
 (segment (start 163.365 101.500001) (end 162.932499 101.067501) (width 0.2) (layer "F.Cu") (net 6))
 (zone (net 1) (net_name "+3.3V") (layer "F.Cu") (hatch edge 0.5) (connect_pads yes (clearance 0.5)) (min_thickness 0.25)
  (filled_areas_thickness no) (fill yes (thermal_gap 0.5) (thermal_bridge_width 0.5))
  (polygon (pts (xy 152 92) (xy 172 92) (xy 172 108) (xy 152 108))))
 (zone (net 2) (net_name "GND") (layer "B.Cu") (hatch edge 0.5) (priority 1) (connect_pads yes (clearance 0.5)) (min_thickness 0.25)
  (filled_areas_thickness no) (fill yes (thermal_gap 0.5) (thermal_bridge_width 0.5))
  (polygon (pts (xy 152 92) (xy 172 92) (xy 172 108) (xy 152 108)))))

